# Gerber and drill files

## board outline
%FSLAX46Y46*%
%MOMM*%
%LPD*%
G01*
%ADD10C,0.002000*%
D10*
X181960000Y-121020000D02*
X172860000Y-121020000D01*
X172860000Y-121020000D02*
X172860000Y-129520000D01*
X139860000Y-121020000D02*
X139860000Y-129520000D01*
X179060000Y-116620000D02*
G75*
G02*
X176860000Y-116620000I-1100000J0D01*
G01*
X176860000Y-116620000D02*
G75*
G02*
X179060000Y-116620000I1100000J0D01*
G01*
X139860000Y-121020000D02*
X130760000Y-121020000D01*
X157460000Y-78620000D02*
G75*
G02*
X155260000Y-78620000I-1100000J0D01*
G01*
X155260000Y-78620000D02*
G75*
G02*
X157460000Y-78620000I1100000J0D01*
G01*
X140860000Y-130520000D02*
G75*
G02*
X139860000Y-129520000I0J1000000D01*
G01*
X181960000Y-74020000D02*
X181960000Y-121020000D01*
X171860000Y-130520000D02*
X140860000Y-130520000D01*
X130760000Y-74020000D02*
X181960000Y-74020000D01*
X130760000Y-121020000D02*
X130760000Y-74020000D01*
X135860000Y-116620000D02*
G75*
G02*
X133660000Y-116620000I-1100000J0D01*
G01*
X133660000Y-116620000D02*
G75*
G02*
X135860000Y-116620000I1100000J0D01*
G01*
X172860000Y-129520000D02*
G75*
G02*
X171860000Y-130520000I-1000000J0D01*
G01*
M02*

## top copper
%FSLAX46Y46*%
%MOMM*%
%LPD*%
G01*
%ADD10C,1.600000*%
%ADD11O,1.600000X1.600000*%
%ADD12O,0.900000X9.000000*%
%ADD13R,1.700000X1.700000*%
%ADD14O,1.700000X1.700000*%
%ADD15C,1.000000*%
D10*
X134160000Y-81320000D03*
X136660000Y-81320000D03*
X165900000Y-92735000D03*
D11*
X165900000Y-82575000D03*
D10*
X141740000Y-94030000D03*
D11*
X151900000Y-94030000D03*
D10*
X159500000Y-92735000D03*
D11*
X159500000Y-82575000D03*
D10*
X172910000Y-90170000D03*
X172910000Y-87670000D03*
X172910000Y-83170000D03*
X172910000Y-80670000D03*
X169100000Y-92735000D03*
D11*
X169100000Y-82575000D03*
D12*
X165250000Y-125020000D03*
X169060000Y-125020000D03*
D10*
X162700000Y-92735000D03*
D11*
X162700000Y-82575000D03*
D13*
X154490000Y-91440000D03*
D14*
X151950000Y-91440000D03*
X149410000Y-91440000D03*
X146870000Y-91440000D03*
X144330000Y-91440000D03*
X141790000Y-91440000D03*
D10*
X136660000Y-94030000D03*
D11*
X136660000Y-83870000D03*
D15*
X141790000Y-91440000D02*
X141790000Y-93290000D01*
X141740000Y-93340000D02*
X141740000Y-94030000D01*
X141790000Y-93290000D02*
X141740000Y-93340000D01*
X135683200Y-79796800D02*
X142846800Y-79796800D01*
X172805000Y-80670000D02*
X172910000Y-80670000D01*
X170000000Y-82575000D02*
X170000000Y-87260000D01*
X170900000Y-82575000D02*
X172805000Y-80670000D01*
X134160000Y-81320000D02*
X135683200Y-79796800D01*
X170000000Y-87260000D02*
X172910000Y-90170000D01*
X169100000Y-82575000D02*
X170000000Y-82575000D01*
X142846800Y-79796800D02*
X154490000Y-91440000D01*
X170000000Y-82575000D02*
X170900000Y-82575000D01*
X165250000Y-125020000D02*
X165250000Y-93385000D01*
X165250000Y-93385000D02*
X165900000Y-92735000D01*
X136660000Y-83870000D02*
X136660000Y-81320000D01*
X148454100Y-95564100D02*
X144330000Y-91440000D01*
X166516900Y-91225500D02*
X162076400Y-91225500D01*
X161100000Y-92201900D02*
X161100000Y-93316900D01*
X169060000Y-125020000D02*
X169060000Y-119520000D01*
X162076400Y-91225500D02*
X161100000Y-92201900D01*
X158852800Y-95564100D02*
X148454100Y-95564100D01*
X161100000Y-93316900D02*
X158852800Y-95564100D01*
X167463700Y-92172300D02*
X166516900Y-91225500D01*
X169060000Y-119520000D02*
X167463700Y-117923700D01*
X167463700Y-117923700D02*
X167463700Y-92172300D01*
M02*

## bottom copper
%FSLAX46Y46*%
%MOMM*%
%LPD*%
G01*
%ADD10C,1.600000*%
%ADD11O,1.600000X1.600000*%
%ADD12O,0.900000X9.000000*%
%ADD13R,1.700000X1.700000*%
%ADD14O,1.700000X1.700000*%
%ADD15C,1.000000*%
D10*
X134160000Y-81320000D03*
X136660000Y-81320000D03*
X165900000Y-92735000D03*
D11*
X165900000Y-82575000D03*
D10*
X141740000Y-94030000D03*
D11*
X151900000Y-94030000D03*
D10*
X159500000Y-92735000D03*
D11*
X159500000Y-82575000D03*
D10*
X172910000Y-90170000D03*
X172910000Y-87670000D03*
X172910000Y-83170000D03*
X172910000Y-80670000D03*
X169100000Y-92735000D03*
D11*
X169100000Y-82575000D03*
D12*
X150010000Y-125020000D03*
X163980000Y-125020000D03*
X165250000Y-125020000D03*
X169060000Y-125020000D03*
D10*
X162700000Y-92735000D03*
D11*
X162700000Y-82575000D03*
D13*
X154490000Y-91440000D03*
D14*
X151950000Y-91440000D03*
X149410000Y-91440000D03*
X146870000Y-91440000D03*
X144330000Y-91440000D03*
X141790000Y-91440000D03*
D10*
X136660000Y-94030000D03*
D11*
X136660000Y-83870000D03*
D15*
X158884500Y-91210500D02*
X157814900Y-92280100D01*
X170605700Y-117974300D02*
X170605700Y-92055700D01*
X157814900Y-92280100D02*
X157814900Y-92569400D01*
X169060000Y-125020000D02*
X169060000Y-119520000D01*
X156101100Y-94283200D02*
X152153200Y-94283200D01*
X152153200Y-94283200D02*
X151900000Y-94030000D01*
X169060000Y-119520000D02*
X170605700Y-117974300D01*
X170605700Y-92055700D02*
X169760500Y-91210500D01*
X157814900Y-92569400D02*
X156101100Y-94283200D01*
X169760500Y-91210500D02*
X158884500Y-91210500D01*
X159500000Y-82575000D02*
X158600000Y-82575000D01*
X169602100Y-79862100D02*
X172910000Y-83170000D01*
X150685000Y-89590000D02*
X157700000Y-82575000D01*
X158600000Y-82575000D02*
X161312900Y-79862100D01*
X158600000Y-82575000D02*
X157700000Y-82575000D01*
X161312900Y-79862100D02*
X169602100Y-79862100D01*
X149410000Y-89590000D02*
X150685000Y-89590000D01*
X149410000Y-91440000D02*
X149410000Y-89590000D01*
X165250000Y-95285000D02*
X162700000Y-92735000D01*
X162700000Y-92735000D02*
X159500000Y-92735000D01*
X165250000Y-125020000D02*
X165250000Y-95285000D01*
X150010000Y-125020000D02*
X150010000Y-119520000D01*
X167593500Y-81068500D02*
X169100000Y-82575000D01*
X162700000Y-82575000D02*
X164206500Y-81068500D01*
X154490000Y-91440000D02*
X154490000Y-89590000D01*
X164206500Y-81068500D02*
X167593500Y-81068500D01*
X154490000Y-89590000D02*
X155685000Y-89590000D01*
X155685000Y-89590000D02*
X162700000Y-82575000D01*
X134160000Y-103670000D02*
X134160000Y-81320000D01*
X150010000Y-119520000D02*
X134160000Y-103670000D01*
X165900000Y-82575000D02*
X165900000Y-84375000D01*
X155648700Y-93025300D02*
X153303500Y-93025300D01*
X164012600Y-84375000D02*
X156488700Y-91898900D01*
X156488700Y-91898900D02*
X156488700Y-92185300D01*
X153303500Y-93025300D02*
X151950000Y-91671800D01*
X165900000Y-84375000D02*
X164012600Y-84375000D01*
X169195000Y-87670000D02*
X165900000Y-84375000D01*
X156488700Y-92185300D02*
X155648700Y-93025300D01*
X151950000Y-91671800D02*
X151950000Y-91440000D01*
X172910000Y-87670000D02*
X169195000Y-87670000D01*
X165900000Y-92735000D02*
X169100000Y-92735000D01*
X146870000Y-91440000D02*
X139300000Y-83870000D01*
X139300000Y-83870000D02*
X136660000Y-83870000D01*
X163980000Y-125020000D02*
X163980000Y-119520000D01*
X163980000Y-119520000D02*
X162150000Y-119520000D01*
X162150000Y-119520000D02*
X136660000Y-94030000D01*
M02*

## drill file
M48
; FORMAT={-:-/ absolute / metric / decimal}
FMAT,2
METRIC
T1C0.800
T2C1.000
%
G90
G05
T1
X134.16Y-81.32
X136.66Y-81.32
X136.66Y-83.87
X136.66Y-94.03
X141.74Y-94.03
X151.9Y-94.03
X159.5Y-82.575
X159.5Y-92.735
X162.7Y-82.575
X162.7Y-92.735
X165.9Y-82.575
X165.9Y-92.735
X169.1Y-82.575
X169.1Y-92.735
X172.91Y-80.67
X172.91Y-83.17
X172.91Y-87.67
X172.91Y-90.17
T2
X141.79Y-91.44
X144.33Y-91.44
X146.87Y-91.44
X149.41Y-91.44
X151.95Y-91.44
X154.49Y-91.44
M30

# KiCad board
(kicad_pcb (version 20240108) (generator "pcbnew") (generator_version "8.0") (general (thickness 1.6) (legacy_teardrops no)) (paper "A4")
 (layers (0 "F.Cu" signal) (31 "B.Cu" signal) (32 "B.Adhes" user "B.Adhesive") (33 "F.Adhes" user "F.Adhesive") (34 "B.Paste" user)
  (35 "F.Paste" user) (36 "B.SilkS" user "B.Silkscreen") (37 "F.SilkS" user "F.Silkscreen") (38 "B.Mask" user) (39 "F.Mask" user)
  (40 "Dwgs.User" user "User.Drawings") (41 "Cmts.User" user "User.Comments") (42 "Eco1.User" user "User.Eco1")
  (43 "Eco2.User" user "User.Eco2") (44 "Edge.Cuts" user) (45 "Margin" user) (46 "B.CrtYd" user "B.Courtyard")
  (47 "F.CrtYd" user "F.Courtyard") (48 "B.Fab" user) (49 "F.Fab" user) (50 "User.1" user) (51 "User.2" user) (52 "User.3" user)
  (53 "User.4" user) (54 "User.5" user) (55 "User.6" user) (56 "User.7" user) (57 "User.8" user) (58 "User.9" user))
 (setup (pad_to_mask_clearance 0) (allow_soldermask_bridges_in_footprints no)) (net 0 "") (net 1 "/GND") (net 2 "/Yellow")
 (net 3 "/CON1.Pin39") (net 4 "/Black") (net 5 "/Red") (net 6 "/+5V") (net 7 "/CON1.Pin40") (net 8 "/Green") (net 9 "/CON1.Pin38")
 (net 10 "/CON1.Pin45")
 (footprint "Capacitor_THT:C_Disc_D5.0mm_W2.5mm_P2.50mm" (layer "F.Cu") (at 134.16 81.32)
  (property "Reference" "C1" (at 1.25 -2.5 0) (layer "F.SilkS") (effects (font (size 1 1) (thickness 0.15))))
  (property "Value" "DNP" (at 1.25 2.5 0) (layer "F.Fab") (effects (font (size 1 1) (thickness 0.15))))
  (pad "1" thru_hole circle (at 0 0) (size 1.6 1.6) (drill 0.8) (layers "*.Cu" "*.Mask") (remove_unused_layers no) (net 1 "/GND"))
  (pad "2" thru_hole circle (at 2.5 0) (size 1.6 1.6) (drill 0.8) (layers "*.Cu" "*.Mask") (remove_unused_layers no) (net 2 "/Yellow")))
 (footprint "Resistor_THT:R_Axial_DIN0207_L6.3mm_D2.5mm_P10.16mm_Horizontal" (layer "F.Cu") (at 165.9 92.735 90)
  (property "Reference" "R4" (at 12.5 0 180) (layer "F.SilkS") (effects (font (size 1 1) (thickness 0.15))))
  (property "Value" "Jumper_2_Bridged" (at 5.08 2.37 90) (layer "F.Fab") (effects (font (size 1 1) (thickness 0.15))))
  (pad "1" thru_hole circle (at 0 0 90) (size 1.6 1.6) (drill 0.8) (layers "*.Cu" "*.Mask") (remove_unused_layers no) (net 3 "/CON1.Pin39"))
  (pad "2" thru_hole oval (at 10.16 0 90) (size 1.6 1.6) (drill 0.8) (layers "*.Cu" "*.Mask") (remove_unused_layers no) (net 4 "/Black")))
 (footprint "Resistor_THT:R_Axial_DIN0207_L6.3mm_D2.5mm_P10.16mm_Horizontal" (layer "F.Cu") (at 141.74 94.03)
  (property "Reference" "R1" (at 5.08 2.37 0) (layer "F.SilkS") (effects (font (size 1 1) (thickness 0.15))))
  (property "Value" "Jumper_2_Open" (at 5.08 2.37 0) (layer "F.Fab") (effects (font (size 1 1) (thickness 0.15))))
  (pad "1" thru_hole circle (at 0 0) (size 1.6 1.6) (drill 0.8) (layers "*.Cu" "*.Mask") (remove_unused_layers no) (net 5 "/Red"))
  (pad "2" thru_hole oval (at 10.16 0) (size 1.6 1.6) (drill 0.8) (layers "*.Cu" "*.Mask") (remove_unused_layers no) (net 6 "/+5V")))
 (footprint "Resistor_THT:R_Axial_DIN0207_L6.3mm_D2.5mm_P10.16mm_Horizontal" (layer "F.Cu") (at 159.5 92.735 90)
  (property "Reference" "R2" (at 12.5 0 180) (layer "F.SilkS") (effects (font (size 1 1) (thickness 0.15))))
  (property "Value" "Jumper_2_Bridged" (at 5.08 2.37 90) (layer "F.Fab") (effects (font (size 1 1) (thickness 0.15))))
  (pad "1" thru_hole circle (at 0 0 90) (size 1.6 1.6) (drill 0.8) (layers "*.Cu" "*.Mask") (remove_unused_layers no) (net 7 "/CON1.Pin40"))
  (pad "2" thru_hole oval (at 10.16 0 90) (size 1.6 1.6) (drill 0.8) (layers "*.Cu" "*.Mask") (remove_unused_layers no) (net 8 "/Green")))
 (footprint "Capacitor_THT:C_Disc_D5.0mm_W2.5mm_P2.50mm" (layer "F.Cu") (at 172.91 90.17 90)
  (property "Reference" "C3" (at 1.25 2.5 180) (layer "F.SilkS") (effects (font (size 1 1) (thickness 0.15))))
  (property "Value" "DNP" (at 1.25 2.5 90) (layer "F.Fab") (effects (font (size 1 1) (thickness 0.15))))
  (pad "1" thru_hole circle (at 0 0 90) (size 1.6 1.6) (drill 0.8) (layers "*.Cu" "*.Mask") (remove_unused_layers no) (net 1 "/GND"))
  (pad "2" thru_hole circle (at 2.5 0 90) (size 1.6 1.6) (drill 0.8) (layers "*.Cu" "*.Mask") (remove_unused_layers no) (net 4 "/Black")))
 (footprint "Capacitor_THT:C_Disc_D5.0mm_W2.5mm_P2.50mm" (layer "F.Cu") (at 172.91 83.17 90)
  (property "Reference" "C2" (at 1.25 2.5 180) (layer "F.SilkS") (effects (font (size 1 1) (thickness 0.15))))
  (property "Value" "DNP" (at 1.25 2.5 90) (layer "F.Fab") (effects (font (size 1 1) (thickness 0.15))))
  (pad "1" thru_hole circle (at 0 0 90) (size 1.6 1.6) (drill 0.8) (layers "*.Cu" "*.Mask") (remove_unused_layers no) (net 8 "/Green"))
  (pad "2" thru_hole circle (at 2.5 0 90) (size 1.6 1.6) (drill 0.8) (layers "*.Cu" "*.Mask") (remove_unused_layers no) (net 1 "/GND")))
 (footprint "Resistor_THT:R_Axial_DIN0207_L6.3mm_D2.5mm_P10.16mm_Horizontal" (layer "F.Cu") (at 169.1 92.735 90)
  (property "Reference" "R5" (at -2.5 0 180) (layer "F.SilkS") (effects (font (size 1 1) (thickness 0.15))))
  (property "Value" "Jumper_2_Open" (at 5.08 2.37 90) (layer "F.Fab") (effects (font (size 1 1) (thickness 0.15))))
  (pad "1" thru_hole circle (at 0 0 90) (size 1.6 1.6) (drill 0.8) (layers "*.Cu" "*.Mask") (remove_unused_layers no) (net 3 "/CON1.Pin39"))
  (pad "2" thru_hole oval (at 10.16 0 90) (size 1.6 1.6) (drill 0.8) (layers "*.Cu" "*.Mask") (remove_unused_layers no) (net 1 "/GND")))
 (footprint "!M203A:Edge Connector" (layer "F.Cu") (at 156.36 125.02)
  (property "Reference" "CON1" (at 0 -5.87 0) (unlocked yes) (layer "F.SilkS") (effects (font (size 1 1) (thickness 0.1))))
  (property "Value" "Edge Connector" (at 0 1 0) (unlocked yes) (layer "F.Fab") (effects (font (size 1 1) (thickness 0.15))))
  (pad "16" smd oval (at -6.35 0 180) (size 0.9 9) (layers "B.Cu" "B.Mask") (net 1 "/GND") (thermal_bridge_angle 45))
  (pad "38" smd oval (at 7.62 0 180) (size 0.9 9) (layers "B.Cu" "B.Mask") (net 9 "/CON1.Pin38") (thermal_bridge_angle 45))
  (pad "39" smd oval (at 8.89 0) (size 0.9 9) (layers "F.Cu" "F.Mask") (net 3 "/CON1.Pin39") (thermal_bridge_angle 45))
  (pad "40" smd oval (at 8.89 0 180) (size 0.9 9) (layers "B.Cu" "B.Mask") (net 7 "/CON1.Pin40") (thermal_bridge_angle 45))
  (pad "45" smd oval (at 12.7 0) (size 0.9 9) (layers "F.Cu" "F.Mask") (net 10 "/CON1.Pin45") (thermal_bridge_angle 45))
  (pad "46" smd oval (at 12.7 0 180) (size 0.9 9) (layers "B.Cu" "B.Mask") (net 6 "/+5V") (thermal_bridge_angle 45)))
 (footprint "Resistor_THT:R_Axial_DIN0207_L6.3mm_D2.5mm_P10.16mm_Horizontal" (layer "F.Cu") (at 162.7 92.735 90)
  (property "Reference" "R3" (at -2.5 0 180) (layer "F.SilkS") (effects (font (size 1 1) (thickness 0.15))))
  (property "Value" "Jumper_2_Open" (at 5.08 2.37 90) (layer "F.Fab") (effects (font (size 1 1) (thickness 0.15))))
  (pad "1" thru_hole circle (at 0 0 90) (size 1.6 1.6) (drill 0.8) (layers "*.Cu" "*.Mask") (remove_unused_layers no) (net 7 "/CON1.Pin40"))
  (pad "2" thru_hole oval (at 10.16 0 90) (size 1.6 1.6) (drill 0.8) (layers "*.Cu" "*.Mask") (remove_unused_layers no) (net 1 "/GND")))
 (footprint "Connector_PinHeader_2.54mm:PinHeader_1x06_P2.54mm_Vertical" (layer "F.Cu") (at 154.49 91.44 -90)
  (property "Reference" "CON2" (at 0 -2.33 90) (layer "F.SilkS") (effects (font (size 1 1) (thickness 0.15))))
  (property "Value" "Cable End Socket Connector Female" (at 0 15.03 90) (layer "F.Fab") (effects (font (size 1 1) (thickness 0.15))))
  (pad "1" thru_hole rect (at 0 0 270) (size 1.7 1.7) (drill 1) (layers "*.Cu" "*.Mask") (remove_unused_layers no) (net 1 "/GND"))
  (pad "2" thru_hole oval (at 0 2.54 270) (size 1.7 1.7) (drill 1) (layers "*.Cu" "*.Mask") (remove_unused_layers no) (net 4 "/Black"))
  (pad "3" thru_hole oval (at 0 5.08 270) (size 1.7 1.7) (drill 1) (layers "*.Cu" "*.Mask") (remove_unused_layers no) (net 8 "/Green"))
  (pad "4" thru_hole oval (at 0 7.62 270) (size 1.7 1.7) (drill 1) (layers "*.Cu" "*.Mask") (remove_unused_layers no) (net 2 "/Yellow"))
  (pad "5" thru_hole oval (at 0 10.16 270) (size 1.7 1.7) (drill 1) (layers "*.Cu" "*.Mask") (remove_unused_layers no)
   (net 10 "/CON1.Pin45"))
  (pad "6" thru_hole oval (at 0 12.7 270) (size 1.7 1.7) (drill 1) (layers "*.Cu" "*.Mask") (remove_unused_layers no) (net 5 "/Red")))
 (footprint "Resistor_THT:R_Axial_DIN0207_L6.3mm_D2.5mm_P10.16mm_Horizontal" (layer "F.Cu") (at 136.66 94.03 90)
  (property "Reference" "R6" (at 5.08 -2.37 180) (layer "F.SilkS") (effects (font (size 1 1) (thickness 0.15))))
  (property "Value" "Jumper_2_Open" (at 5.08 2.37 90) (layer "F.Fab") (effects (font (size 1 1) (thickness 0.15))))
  (pad "1" thru_hole circle (at 0 0 90) (size 1.6 1.6) (drill 0.8) (layers "*.Cu" "*.Mask") (remove_unused_layers no) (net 9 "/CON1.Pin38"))
  (pad "2" thru_hole oval (at 10.16 0 90) (size 1.6 1.6) (drill 0.8) (layers "*.Cu" "*.Mask") (remove_unused_layers no) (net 2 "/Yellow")))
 (gr_line (start 181.96 121.02) (end 172.86 121.02) (stroke (width 0.002) (type default)) (layer "Edge.Cuts"))
 (gr_line (start 172.86 121.02) (end 172.86 129.52) (stroke (width 0.002) (type default)) (layer "Edge.Cuts"))
 (gr_line (start 139.86 121.02) (end 139.86 129.52) (stroke (width 0.002) (type default)) (layer "Edge.Cuts"))
 (gr_circle (center 177.96 116.62) (end 179.06 116.62) (stroke (width 0.002) (type default)) (fill none) (layer "Edge.Cuts"))
 (gr_line (start 139.86 121.02) (end 130.76 121.02) (stroke (width 0.002) (type default)) (layer "Edge.Cuts"))
 (gr_circle (center 156.36 78.62) (end 157.46 78.62) (stroke (width 0.002) (type default)) (fill none) (layer "Edge.Cuts"))
 (gr_arc (start 140.86 130.52) (mid 140.152893 130.227107) (end 139.86 129.52) (stroke (width 0.002) (type default)) (layer "Edge.Cuts"))
 (gr_line (start 181.96 74.02) (end 181.96 121.02) (stroke (width 0.002) (type default)) (layer "Edge.Cuts"))
 (gr_line (start 171.86 130.52) (end 140.86 130.52) (stroke (width 0.002) (type default)) (layer "Edge.Cuts"))
 (gr_line (start 130.76 74.02) (end 181.96 74.02) (stroke (width 0.002) (type default)) (layer "Edge.Cuts"))
 (gr_line (start 130.76 121.02) (end 130.76 74.02) (stroke (width 0.002) (type default)) (layer "Edge.Cuts"))
 (gr_circle (center 134.76 116.62) (end 135.86 116.62) (stroke (width 0.002) (type default)) (fill none) (layer "Edge.Cuts"))
 (gr_arc (start 172.86 129.52) (mid 172.567107 130.227107) (end 171.86 130.52) (stroke (width 0.002) (type default)) (layer "Edge.Cuts"))
 (segment (start 158.8845 91.2105) (end 157.8149 92.2801) (width 1) (layer "B.Cu") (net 6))
 (segment (start 170.6057 117.9743) (end 170.6057 92.0557) (width 1) (layer "B.Cu") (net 6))
 (segment (start 157.8149 92.2801) (end 157.8149 92.5694) (width 1) (layer "B.Cu") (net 6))
 (segment (start 169.06 125.02) (end 169.06 119.52) (width 1) (layer "B.Cu") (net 6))
 (segment (start 156.1011 94.2832) (end 152.1532 94.2832) (width 1) (layer "B.Cu") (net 6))
 (segment (start 152.1532 94.2832) (end 151.9 94.03) (width 1) (layer "B.Cu") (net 6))
 (segment (start 169.06 119.52) (end 170.6057 117.9743) (width 1) (layer "B.Cu") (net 6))
 (segment (start 170.6057 92.0557) (end 169.7605 91.2105) (width 1) (layer "B.Cu") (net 6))
 (segment (start 157.8149 92.5694) (end 156.1011 94.2832) (width 1) (layer "B.Cu") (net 6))
 (segment (start 169.7605 91.2105) (end 158.8845 91.2105) (width 1) (layer "B.Cu") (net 6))
 (segment (start 141.79 91.44) (end 141.79 93.29) (width 1) (layer "F.Cu") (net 5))
 (segment (start 141.74 93.34) (end 141.74 94.03) (width 1) (layer "F.Cu") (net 5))
 (segment (start 141.79 93.29) (end 141.74 93.34) (width 1) (layer "F.Cu") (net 5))
 (segment (start 159.5 82.575) (end 158.6 82.575) (width 1) (layer "B.Cu") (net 8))
 (segment (start 169.6021 79.8621) (end 172.91 83.17) (width 1) (layer "B.Cu") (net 8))
 (segment (start 150.685 89.59) (end 157.7 82.575) (width 1) (layer "B.Cu") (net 8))
 (segment (start 158.6 82.575) (end 161.3129 79.8621) (width 1) (layer "B.Cu") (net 8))
 (segment (start 158.6 82.575) (end 157.7 82.575) (width 1) (layer "B.Cu") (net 8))
 (segment (start 161.3129 79.8621) (end 169.6021 79.8621) (width 1) (layer "B.Cu") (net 8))
 (segment (start 149.41 89.59) (end 150.685 89.59) (width 1) (layer "B.Cu") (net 8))
 (segment (start 149.41 91.44) (end 149.41 89.59) (width 1) (layer "B.Cu") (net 8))
 (segment (start 165.25 95.285) (end 162.7 92.735) (width 1) (layer "B.Cu") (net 7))
 (segment (start 162.7 92.735) (end 159.5 92.735) (width 1) (layer "B.Cu") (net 7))
 (segment (start 165.25 125.02) (end 165.25 95.285) (width 1) (layer "B.Cu") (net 7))
 (segment (start 135.6832 79.7968) (end 142.8468 79.7968) (width 1) (layer "F.Cu") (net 1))
 (segment (start 172.805 80.67) (end 172.91 80.67) (width 1) (layer "F.Cu") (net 1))
 (segment (start 170 82.575) (end 170 87.26) (width 1) (layer "F.Cu") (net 1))
 (segment (start 170.9 82.575) (end 172.805 80.67) (width 1) (layer "F.Cu") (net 1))
 (segment (start 134.16 81.32) (end 135.6832 79.7968) (width 1) (layer "F.Cu") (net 1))
 (segment (start 170 87.26) (end 172.91 90.17) (width 1) (layer "F.Cu") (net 1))
 (segment (start 169.1 82.575) (end 170 82.575) (width 1) (layer "F.Cu") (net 1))
 (segment (start 142.8468 79.7968) (end 154.49 91.44) (width 1) (layer "F.Cu") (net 1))
 (segment (start 170 82.575) (end 170.9 82.575) (width 1) (layer "F.Cu") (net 1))
 (segment (start 150.01 125.02) (end 150.01 119.52) (width 1) (layer "B.Cu") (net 1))
 (segment (start 167.5935 81.0685) (end 169.1 82.575) (width 1) (layer "B.Cu") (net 1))
 (segment (start 162.7 82.575) (end 164.2065 81.0685) (width 1) (layer "B.Cu") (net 1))
 (segment (start 154.49 91.44) (end 154.49 89.59) (width 1) (layer "B.Cu") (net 1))
 (segment (start 164.2065 81.0685) (end 167.5935 81.0685) (width 1) (layer "B.Cu") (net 1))
 (segment (start 154.49 89.59) (end 155.685 89.59) (width 1) (layer "B.Cu") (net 1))
 (segment (start 155.685 89.59) (end 162.7 82.575) (width 1) (layer "B.Cu") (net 1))
 (segment (start 134.16 103.67) (end 134.16 81.32) (width 1) (layer "B.Cu") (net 1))
 (segment (start 150.01 119.52) (end 134.16 103.67) (width 1) (layer "B.Cu") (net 1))
 (segment (start 165.9 82.575) (end 165.9 84.375) (width 1) (layer "B.Cu") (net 4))
 (segment (start 155.6487 93.0253) (end 153.3035 93.0253) (width 1) (layer "B.Cu") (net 4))
 (segment (start 164.0126 84.375) (end 156.4887 91.8989) (width 1) (layer "B.Cu") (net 4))
 (segment (start 156.4887 91.8989) (end 156.4887 92.1853) (width 1) (layer "B.Cu") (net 4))
 (segment (start 153.3035 93.0253) (end 151.95 91.6718) (width 1) (layer "B.Cu") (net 4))
 (segment (start 165.9 84.375) (end 164.0126 84.375) (width 1) (layer "B.Cu") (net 4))
 (segment (start 169.195 87.67) (end 165.9 84.375) (width 1) (layer "B.Cu") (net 4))
 (segment (start 156.4887 92.1853) (end 155.6487 93.0253) (width 1) (layer "B.Cu") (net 4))
 (segment (start 151.95 91.6718) (end 151.95 91.44) (width 1) (layer "B.Cu") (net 4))
 (segment (start 172.91 87.67) (end 169.195 87.67) (width 1) (layer "B.Cu") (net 4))
 (segment (start 165.25 125.02) (end 165.25 93.385) (width 1) (layer "F.Cu") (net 3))
 (segment (start 165.25 93.385) (end 165.9 92.735) (width 1) (layer "F.Cu") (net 3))
 (segment (start 165.9 92.735) (end 169.1 92.735) (width 1) (layer "B.Cu") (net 3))
 (segment (start 136.66 83.87) (end 136.66 81.32) (width 1) (layer "F.Cu") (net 2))
 (segment (start 146.87 91.44) (end 139.3 83.87) (width 1) (layer "B.Cu") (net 2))
 (segment (start 139.3 83.87) (end 136.66 83.87) (width 1) (layer "B.Cu") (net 2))
 (segment (start 163.98 125.02) (end 163.98 119.52) (width 1) (layer "B.Cu") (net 9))
 (segment (start 163.98 119.52) (end 162.15 119.52) (width 1) (layer "B.Cu") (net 9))
 (segment (start 162.15 119.52) (end 136.66 94.03) (width 1) (layer "B.Cu") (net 9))
 (segment (start 148.4541 95.5641) (end 144.33 91.44) (width 1) (layer "F.Cu") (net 10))
 (segment (start 166.5169 91.2255) (end 162.0764 91.2255) (width 1) (layer "F.Cu") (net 10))
 (segment (start 161.1 92.2019) (end 161.1 93.3169) (width 1) (layer "F.Cu") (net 10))
 (segment (start 169.06 125.02) (end 169.06 119.52) (width 1) (layer "F.Cu") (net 10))
 (segment (start 162.0764 91.2255) (end 161.1 92.2019) (width 1) (layer "F.Cu") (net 10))
 (segment (start 158.8528 95.5641) (end 148.4541 95.5641) (width 1) (layer "F.Cu") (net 10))
 (segment (start 161.1 93.3169) (end 158.8528 95.5641) (width 1) (layer "F.Cu") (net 10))
 (segment (start 167.4637 92.1723) (end 166.5169 91.2255) (width 1) (layer "F.Cu") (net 10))
 (segment (start 169.06 119.52) (end 167.4637 117.9237) (width 1) (layer "F.Cu") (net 10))
 (segment (start 167.4637 117.9237) (end 167.4637 92.1723) (width 1) (layer "F.Cu") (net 10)))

